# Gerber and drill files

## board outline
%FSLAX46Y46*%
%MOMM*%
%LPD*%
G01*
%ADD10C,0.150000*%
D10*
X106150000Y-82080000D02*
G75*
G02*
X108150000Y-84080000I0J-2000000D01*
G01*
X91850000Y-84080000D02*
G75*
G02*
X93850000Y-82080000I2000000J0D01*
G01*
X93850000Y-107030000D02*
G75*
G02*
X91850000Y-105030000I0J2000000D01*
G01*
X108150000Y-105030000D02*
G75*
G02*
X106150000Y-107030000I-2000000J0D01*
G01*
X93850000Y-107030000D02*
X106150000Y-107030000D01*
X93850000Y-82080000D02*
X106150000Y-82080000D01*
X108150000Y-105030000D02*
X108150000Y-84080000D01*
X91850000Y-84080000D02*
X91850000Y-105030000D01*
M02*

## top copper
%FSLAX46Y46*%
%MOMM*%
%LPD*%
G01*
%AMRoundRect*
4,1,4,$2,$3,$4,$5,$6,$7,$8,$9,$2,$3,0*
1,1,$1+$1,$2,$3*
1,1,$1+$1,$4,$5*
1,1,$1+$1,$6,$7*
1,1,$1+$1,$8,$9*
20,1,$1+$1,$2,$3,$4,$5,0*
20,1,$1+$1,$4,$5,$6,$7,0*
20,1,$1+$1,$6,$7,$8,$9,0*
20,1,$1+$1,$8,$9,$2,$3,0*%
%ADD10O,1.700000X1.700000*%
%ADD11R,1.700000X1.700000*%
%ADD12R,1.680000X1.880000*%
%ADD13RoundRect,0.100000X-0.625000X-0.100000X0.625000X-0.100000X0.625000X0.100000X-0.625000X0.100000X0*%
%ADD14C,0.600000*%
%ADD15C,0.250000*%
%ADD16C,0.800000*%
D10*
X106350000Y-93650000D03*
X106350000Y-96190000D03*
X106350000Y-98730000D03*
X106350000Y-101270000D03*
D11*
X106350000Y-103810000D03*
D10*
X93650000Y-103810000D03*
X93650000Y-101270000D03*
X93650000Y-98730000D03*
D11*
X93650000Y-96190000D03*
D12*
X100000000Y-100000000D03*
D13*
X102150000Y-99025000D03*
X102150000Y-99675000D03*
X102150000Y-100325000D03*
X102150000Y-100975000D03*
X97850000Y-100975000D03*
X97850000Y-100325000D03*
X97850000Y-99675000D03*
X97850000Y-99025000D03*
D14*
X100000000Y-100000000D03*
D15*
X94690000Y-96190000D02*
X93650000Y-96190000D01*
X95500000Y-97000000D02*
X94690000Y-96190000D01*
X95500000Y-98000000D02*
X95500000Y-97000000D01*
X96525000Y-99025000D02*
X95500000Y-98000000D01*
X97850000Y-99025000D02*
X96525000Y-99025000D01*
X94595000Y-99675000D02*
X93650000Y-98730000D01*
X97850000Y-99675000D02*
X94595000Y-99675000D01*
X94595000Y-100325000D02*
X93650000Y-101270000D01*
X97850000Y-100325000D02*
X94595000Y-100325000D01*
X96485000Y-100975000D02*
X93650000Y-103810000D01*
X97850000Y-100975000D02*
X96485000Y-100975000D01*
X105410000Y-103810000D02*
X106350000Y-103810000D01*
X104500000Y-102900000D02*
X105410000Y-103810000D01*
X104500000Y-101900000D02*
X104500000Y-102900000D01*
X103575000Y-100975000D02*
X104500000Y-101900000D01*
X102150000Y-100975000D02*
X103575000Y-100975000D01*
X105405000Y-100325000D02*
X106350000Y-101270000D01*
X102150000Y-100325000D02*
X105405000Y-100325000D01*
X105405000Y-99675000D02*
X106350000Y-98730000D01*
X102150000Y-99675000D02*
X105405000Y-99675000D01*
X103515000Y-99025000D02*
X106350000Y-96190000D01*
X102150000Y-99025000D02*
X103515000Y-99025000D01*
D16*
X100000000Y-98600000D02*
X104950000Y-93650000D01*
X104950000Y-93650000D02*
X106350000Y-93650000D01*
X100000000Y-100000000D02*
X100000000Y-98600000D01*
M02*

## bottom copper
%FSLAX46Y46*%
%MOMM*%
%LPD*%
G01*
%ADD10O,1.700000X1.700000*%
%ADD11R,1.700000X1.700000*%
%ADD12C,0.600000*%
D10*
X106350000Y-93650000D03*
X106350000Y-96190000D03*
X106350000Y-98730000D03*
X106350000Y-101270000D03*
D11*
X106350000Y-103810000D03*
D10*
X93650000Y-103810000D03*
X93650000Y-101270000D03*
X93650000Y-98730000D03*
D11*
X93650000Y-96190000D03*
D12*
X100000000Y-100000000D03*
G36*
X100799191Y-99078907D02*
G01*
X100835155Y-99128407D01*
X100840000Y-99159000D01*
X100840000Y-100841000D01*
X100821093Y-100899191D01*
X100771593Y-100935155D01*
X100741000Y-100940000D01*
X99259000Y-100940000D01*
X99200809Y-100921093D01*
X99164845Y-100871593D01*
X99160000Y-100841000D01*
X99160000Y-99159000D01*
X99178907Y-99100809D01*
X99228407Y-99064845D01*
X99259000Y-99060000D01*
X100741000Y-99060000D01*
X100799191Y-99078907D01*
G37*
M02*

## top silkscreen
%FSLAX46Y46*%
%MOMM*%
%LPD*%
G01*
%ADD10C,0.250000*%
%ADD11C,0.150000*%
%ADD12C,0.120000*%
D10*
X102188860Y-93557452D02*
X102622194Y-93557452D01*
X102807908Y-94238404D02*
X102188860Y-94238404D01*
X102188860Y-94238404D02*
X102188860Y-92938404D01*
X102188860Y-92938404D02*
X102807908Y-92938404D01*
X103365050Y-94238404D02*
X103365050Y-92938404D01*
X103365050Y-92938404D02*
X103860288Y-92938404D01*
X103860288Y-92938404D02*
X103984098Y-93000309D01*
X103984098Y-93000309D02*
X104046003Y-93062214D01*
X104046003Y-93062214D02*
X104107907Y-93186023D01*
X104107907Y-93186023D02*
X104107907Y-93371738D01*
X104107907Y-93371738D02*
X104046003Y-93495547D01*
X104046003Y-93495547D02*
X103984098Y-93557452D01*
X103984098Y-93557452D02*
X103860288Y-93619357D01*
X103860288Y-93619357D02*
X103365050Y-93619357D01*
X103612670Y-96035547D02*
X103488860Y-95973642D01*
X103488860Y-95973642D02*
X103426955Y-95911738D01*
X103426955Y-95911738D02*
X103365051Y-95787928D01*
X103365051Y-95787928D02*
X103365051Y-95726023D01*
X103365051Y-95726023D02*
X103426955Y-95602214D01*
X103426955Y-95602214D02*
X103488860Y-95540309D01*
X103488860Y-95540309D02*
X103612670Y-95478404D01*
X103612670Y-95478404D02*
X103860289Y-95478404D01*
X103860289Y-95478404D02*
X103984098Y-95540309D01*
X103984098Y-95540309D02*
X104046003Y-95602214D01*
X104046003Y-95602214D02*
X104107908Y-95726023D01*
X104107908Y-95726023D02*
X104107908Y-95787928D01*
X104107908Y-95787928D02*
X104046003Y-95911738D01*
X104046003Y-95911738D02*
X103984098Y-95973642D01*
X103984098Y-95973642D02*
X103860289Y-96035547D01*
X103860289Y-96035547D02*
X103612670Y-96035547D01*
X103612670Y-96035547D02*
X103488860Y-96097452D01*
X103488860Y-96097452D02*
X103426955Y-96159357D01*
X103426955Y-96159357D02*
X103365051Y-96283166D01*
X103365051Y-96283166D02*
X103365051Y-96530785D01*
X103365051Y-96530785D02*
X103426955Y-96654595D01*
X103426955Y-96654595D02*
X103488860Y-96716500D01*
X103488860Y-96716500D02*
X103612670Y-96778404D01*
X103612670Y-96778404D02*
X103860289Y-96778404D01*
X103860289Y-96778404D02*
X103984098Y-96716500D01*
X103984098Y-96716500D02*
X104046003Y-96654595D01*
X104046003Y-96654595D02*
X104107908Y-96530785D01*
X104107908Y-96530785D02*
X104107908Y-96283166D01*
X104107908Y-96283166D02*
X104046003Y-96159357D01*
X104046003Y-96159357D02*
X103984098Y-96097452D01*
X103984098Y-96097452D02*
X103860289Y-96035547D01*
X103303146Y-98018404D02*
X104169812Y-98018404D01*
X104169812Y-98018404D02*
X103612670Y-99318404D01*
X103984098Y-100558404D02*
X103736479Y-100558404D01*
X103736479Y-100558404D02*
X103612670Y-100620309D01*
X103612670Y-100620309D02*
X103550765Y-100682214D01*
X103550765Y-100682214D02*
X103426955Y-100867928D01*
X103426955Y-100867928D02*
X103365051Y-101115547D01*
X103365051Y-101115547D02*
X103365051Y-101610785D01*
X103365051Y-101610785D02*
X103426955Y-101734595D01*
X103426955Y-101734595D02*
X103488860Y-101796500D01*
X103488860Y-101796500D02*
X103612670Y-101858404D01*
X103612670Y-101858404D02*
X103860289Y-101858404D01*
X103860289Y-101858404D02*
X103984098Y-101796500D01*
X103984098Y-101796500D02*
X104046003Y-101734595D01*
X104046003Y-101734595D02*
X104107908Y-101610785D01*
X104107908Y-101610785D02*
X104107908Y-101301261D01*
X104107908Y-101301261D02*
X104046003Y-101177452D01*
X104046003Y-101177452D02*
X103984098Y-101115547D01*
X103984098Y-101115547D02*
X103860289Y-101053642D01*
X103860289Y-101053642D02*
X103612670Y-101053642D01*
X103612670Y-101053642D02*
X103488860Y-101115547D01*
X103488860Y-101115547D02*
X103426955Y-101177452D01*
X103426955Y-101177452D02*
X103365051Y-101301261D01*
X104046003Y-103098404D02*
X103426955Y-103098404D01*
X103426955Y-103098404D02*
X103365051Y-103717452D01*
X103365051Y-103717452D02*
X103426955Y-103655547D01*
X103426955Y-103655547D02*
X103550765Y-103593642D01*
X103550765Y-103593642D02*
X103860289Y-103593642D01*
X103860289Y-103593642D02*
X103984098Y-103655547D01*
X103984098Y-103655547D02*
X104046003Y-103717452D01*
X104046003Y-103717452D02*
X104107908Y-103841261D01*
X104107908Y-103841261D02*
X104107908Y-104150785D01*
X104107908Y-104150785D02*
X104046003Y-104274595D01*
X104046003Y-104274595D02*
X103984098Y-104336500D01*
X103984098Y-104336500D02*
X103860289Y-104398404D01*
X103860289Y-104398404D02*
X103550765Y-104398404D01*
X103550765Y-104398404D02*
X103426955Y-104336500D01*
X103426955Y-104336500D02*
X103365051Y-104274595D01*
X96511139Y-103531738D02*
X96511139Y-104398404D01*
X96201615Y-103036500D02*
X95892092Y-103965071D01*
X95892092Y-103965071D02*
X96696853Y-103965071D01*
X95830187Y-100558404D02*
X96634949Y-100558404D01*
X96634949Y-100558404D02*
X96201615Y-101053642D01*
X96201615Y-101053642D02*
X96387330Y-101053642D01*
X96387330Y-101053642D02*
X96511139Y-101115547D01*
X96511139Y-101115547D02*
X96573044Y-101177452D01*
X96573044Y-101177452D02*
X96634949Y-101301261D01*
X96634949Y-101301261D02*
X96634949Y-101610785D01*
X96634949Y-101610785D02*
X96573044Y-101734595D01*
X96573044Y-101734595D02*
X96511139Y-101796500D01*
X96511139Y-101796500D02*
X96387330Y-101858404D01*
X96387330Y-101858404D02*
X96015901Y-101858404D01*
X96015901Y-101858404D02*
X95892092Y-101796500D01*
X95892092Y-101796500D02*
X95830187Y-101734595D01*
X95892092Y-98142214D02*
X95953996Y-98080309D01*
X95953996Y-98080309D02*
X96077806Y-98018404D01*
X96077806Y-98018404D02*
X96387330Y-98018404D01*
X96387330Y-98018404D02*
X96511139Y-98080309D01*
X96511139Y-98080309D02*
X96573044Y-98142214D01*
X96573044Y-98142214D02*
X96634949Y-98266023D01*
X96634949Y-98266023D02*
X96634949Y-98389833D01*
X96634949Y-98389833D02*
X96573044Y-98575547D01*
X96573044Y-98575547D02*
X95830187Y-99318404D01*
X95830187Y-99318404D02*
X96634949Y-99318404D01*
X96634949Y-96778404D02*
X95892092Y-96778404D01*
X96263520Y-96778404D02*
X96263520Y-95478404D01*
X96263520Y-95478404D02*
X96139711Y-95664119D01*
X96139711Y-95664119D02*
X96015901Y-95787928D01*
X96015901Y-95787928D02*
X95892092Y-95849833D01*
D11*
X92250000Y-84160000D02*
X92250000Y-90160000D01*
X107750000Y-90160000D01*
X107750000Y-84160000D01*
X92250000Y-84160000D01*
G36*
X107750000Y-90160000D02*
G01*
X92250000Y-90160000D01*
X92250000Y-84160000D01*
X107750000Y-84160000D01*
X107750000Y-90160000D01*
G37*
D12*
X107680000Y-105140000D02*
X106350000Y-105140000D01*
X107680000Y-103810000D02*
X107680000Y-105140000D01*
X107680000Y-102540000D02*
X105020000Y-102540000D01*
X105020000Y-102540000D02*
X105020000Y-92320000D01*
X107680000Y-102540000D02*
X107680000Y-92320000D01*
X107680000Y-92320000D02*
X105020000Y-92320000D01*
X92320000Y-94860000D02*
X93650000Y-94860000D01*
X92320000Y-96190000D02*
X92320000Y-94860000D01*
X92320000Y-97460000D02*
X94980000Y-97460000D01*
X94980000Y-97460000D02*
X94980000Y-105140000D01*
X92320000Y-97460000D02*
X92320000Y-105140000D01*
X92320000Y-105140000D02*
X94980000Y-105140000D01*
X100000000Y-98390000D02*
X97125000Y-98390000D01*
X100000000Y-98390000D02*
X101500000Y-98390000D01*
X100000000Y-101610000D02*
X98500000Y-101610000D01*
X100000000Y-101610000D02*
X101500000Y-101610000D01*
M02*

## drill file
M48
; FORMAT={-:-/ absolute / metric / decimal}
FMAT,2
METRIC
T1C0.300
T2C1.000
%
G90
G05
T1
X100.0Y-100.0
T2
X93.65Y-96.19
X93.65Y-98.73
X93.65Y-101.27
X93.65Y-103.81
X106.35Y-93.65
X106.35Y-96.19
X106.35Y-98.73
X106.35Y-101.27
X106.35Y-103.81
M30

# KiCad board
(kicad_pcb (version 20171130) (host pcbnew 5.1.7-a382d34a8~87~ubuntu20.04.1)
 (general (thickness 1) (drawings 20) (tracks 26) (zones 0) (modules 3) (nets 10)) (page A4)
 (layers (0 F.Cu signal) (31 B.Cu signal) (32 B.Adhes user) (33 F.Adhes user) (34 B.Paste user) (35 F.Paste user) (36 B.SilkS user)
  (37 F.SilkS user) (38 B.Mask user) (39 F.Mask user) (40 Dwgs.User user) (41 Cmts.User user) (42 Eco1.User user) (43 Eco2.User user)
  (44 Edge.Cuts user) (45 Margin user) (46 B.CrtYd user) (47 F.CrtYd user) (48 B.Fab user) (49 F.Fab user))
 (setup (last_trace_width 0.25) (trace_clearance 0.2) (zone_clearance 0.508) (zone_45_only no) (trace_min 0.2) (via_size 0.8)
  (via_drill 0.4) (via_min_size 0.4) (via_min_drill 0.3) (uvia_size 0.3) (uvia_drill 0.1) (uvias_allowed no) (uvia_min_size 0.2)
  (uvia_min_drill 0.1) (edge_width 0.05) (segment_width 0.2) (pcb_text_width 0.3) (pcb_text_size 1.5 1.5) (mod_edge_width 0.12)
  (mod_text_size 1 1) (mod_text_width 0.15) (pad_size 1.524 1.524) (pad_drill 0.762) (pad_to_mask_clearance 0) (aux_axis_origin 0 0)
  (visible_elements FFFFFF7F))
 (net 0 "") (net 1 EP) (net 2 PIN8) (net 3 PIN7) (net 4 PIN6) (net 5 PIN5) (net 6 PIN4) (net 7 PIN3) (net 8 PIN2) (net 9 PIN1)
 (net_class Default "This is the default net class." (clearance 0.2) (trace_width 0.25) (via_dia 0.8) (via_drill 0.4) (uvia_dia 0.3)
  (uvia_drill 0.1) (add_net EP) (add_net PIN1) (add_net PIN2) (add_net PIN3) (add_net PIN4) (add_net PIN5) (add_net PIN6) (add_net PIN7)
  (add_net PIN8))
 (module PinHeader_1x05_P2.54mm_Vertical (layer F.Cu) (at 106.35 103.81 180)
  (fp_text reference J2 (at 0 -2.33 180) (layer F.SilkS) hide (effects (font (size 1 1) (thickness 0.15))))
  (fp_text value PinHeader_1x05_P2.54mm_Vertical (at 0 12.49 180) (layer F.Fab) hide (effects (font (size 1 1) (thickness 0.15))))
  (fp_line (start -1.33 -1.33) (end 0 -1.33) (layer F.SilkS) (width 0.12))
  (fp_line (start -1.33 0) (end -1.33 -1.33) (layer F.SilkS) (width 0.12))
  (fp_line (start -1.33 1.27) (end 1.33 1.27) (layer F.SilkS) (width 0.12))
  (fp_line (start 1.33 1.27) (end 1.33 11.49) (layer F.SilkS) (width 0.12))
  (fp_line (start -1.33 1.27) (end -1.33 11.49) (layer F.SilkS) (width 0.12))
  (fp_line (start -1.33 11.49) (end 1.33 11.49) (layer F.SilkS) (width 0.12))
  (pad 5 thru_hole oval (at 0 10.16 180) (size 1.7 1.7) (drill 1) (layers *.Cu *.Mask) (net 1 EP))
  (pad 4 thru_hole oval (at 0 7.62 180) (size 1.7 1.7) (drill 1) (layers *.Cu *.Mask) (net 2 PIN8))
  (pad 3 thru_hole oval (at 0 5.08 180) (size 1.7 1.7) (drill 1) (layers *.Cu *.Mask) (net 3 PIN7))
  (pad 2 thru_hole oval (at 0 2.54 180) (size 1.7 1.7) (drill 1) (layers *.Cu *.Mask) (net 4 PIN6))
  (pad 1 thru_hole rect (at 0 0 180) (size 1.7 1.7) (drill 1) (layers *.Cu *.Mask) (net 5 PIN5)))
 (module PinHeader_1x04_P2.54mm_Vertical (layer F.Cu) (at 93.65 96.19)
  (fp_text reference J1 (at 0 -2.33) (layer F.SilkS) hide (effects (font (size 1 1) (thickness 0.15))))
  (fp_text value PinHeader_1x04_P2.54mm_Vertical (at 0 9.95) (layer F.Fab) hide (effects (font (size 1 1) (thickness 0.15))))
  (fp_line (start -1.33 -1.33) (end 0 -1.33) (layer F.SilkS) (width 0.12))
  (fp_line (start -1.33 0) (end -1.33 -1.33) (layer F.SilkS) (width 0.12))
  (fp_line (start -1.33 1.27) (end 1.33 1.27) (layer F.SilkS) (width 0.12))
  (fp_line (start 1.33 1.27) (end 1.33 8.95) (layer F.SilkS) (width 0.12))
  (fp_line (start -1.33 1.27) (end -1.33 8.95) (layer F.SilkS) (width 0.12))
  (fp_line (start -1.33 8.95) (end 1.33 8.95) (layer F.SilkS) (width 0.12))
  (pad 4 thru_hole oval (at 0 7.62) (size 1.7 1.7) (drill 1) (layers *.Cu *.Mask) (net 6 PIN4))
  (pad 3 thru_hole oval (at 0 5.08) (size 1.7 1.7) (drill 1) (layers *.Cu *.Mask) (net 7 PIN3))
  (pad 2 thru_hole oval (at 0 2.54) (size 1.7 1.7) (drill 1) (layers *.Cu *.Mask) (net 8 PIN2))
  (pad 1 thru_hole rect (at 0 0) (size 1.7 1.7) (drill 1) (layers *.Cu *.Mask) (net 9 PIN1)))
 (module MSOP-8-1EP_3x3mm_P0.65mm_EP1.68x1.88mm (layer F.Cu) (at 100 100)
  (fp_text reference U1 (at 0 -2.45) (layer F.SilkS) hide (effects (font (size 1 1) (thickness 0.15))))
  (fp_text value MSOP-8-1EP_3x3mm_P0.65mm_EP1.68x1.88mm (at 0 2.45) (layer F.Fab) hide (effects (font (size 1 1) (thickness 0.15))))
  (fp_line (start 0 -1.61) (end -2.875 -1.61) (layer F.SilkS) (width 0.12))
  (fp_line (start 0 -1.61) (end 1.5 -1.61) (layer F.SilkS) (width 0.12))
  (fp_line (start 0 1.61) (end -1.5 1.61) (layer F.SilkS) (width 0.12))
  (fp_line (start 0 1.61) (end 1.5 1.61) (layer F.SilkS) (width 0.12))
  (pad "" smd roundrect (at 0.42 0.47) (size 0.68 0.76) (layers F.Paste) (roundrect_rratio 0.25))
  (pad "" smd roundrect (at 0.42 -0.47) (size 0.68 0.76) (layers F.Paste) (roundrect_rratio 0.25))
  (pad "" smd roundrect (at -0.42 0.47) (size 0.68 0.76) (layers F.Paste) (roundrect_rratio 0.25))
  (pad "" smd roundrect (at -0.42 -0.47) (size 0.68 0.76) (layers F.Paste) (roundrect_rratio 0.25))
  (pad 9 smd rect (at 0 0) (size 1.68 1.88) (layers F.Cu F.Mask) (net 1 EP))
  (pad 8 smd roundrect (at 2.15 -0.975) (size 1.45 0.4) (layers F.Cu F.Paste F.Mask) (roundrect_rratio 0.25) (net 2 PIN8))
  (pad 7 smd roundrect (at 2.15 -0.325) (size 1.45 0.4) (layers F.Cu F.Paste F.Mask) (roundrect_rratio 0.25) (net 3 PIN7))
  (pad 6 smd roundrect (at 2.15 0.325) (size 1.45 0.4) (layers F.Cu F.Paste F.Mask) (roundrect_rratio 0.25) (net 4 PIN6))
  (pad 5 smd roundrect (at 2.15 0.975) (size 1.45 0.4) (layers F.Cu F.Paste F.Mask) (roundrect_rratio 0.25) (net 5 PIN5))
  (pad 4 smd roundrect (at -2.15 0.975) (size 1.45 0.4) (layers F.Cu F.Paste F.Mask) (roundrect_rratio 0.25) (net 6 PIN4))
  (pad 3 smd roundrect (at -2.15 0.325) (size 1.45 0.4) (layers F.Cu F.Paste F.Mask) (roundrect_rratio 0.25) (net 7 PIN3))
  (pad 2 smd roundrect (at -2.15 -0.325) (size 1.45 0.4) (layers F.Cu F.Paste F.Mask) (roundrect_rratio 0.25) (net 8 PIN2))
  (pad 1 smd roundrect (at -2.15 -0.975) (size 1.45 0.4) (layers F.Cu F.Paste F.Mask) (roundrect_rratio 0.25) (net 9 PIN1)))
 (gr_arc (start 106.15 84.08) (end 106.15 82.08) (angle 90) (layer Edge.Cuts) (width 0.15))
 (gr_arc (start 93.85 84.08) (end 91.85 84.08) (angle 90) (layer Edge.Cuts) (width 0.15))
 (gr_arc (start 93.85 105.03) (end 93.85 107.03) (angle 90) (layer Edge.Cuts) (width 0.15))
 (gr_arc (start 106.15 105.03) (end 108.15 105.03) (angle 90) (layer Edge.Cuts) (width 0.15))
 (gr_line (start 93.85 107.03) (end 106.15 107.03) (layer Edge.Cuts) (width 0.15))
 (gr_line (start 93.85 82.08) (end 106.15 82.08) (layer Edge.Cuts) (width 0.15))
 (gr_line (start 108.15 105.03) (end 108.15 84.08) (layer Edge.Cuts) (width 0.15))
 (gr_line (start 91.85 84.08) (end 91.85 105.03) (layer Edge.Cuts) (width 0.15))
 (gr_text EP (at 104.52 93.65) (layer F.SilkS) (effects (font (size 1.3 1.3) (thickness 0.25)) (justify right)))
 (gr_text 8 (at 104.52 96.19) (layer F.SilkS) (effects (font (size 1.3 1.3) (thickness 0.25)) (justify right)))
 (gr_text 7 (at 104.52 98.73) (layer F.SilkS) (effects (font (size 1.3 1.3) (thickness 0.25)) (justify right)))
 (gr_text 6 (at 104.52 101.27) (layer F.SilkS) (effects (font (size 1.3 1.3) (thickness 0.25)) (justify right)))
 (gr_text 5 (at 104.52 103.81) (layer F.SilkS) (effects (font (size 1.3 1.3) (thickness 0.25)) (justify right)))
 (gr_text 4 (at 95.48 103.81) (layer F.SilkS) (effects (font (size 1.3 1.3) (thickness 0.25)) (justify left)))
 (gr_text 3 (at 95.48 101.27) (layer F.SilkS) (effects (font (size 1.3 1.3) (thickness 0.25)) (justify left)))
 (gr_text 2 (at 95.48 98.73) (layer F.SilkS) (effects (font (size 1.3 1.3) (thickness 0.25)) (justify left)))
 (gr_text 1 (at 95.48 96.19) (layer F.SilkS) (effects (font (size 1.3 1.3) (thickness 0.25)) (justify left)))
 (gr_poly (pts (xy 92.25 84.16) (xy 92.25 90.16) (xy 107.75 90.16) (xy 107.75 84.16)) (layer F.SilkS) (width 0.15))
 (segment (start 94.69 96.19) (end 93.65 96.19) (width 0.25) (layer F.Cu) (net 9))
 (segment (start 95.5 97) (end 94.69 96.19) (width 0.25) (layer F.Cu) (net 9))
 (segment (start 95.5 98) (end 95.5 97) (width 0.25) (layer F.Cu) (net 9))
 (segment (start 96.525 99.025) (end 95.5 98) (width 0.25) (layer F.Cu) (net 9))
 (segment (start 97.85 99.025) (end 96.525 99.025) (width 0.25) (layer F.Cu) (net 9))
 (segment (start 94.595 99.675) (end 93.65 98.73) (width 0.25) (layer F.Cu) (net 8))
 (segment (start 97.85 99.675) (end 94.595 99.675) (width 0.25) (layer F.Cu) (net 8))
 (segment (start 94.595 100.325) (end 93.65 101.27) (width 0.25) (layer F.Cu) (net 7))
 (segment (start 97.85 100.325) (end 94.595 100.325) (width 0.25) (layer F.Cu) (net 7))
 (segment (start 96.485 100.975) (end 93.65 103.81) (width 0.25) (layer F.Cu) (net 6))
 (segment (start 97.85 100.975) (end 96.485 100.975) (width 0.25) (layer F.Cu) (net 6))
 (segment (start 105.41 103.81) (end 106.35 103.81) (width 0.25) (layer F.Cu) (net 5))
 (segment (start 104.5 102.9) (end 105.41 103.81) (width 0.25) (layer F.Cu) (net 5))
 (segment (start 104.5 101.9) (end 104.5 102.9) (width 0.25) (layer F.Cu) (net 5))
 (segment (start 103.575 100.975) (end 104.5 101.9) (width 0.25) (layer F.Cu) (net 5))
 (segment (start 102.15 100.975) (end 103.575 100.975) (width 0.25) (layer F.Cu) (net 5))
 (segment (start 105.405 100.325) (end 106.35 101.27) (width 0.25) (layer F.Cu) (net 4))
 (segment (start 102.15 100.325) (end 105.405 100.325) (width 0.25) (layer F.Cu) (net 4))
 (segment (start 105.405 99.675) (end 106.35 98.73) (width 0.25) (layer F.Cu) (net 3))
 (segment (start 102.15 99.675) (end 105.405 99.675) (width 0.25) (layer F.Cu) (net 3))
 (segment (start 103.515 99.025) (end 106.35 96.19) (width 0.25) (layer F.Cu) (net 2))
 (segment (start 102.15 99.025) (end 103.515 99.025) (width 0.25) (layer F.Cu) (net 2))
 (via (at 100 100) (size 0.6) (drill 0.3) (layers F.Cu B.Cu) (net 1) (status 1000000))
 (segment (start 100 98.6) (end 104.95 93.65) (width 0.8) (layer F.Cu) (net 1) (status 1000000))
 (segment (start 104.95 93.65) (end 106.35 93.65) (width 0.8) (layer F.Cu) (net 1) (status 1000000))
 (segment (start 100 100) (end 100 98.6) (width 0.8) (layer F.Cu) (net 1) (status 1000000))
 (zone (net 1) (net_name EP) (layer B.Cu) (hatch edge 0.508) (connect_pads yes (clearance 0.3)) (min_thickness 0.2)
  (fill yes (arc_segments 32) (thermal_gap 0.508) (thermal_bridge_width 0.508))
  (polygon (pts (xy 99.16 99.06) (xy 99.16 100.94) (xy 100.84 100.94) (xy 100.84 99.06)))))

